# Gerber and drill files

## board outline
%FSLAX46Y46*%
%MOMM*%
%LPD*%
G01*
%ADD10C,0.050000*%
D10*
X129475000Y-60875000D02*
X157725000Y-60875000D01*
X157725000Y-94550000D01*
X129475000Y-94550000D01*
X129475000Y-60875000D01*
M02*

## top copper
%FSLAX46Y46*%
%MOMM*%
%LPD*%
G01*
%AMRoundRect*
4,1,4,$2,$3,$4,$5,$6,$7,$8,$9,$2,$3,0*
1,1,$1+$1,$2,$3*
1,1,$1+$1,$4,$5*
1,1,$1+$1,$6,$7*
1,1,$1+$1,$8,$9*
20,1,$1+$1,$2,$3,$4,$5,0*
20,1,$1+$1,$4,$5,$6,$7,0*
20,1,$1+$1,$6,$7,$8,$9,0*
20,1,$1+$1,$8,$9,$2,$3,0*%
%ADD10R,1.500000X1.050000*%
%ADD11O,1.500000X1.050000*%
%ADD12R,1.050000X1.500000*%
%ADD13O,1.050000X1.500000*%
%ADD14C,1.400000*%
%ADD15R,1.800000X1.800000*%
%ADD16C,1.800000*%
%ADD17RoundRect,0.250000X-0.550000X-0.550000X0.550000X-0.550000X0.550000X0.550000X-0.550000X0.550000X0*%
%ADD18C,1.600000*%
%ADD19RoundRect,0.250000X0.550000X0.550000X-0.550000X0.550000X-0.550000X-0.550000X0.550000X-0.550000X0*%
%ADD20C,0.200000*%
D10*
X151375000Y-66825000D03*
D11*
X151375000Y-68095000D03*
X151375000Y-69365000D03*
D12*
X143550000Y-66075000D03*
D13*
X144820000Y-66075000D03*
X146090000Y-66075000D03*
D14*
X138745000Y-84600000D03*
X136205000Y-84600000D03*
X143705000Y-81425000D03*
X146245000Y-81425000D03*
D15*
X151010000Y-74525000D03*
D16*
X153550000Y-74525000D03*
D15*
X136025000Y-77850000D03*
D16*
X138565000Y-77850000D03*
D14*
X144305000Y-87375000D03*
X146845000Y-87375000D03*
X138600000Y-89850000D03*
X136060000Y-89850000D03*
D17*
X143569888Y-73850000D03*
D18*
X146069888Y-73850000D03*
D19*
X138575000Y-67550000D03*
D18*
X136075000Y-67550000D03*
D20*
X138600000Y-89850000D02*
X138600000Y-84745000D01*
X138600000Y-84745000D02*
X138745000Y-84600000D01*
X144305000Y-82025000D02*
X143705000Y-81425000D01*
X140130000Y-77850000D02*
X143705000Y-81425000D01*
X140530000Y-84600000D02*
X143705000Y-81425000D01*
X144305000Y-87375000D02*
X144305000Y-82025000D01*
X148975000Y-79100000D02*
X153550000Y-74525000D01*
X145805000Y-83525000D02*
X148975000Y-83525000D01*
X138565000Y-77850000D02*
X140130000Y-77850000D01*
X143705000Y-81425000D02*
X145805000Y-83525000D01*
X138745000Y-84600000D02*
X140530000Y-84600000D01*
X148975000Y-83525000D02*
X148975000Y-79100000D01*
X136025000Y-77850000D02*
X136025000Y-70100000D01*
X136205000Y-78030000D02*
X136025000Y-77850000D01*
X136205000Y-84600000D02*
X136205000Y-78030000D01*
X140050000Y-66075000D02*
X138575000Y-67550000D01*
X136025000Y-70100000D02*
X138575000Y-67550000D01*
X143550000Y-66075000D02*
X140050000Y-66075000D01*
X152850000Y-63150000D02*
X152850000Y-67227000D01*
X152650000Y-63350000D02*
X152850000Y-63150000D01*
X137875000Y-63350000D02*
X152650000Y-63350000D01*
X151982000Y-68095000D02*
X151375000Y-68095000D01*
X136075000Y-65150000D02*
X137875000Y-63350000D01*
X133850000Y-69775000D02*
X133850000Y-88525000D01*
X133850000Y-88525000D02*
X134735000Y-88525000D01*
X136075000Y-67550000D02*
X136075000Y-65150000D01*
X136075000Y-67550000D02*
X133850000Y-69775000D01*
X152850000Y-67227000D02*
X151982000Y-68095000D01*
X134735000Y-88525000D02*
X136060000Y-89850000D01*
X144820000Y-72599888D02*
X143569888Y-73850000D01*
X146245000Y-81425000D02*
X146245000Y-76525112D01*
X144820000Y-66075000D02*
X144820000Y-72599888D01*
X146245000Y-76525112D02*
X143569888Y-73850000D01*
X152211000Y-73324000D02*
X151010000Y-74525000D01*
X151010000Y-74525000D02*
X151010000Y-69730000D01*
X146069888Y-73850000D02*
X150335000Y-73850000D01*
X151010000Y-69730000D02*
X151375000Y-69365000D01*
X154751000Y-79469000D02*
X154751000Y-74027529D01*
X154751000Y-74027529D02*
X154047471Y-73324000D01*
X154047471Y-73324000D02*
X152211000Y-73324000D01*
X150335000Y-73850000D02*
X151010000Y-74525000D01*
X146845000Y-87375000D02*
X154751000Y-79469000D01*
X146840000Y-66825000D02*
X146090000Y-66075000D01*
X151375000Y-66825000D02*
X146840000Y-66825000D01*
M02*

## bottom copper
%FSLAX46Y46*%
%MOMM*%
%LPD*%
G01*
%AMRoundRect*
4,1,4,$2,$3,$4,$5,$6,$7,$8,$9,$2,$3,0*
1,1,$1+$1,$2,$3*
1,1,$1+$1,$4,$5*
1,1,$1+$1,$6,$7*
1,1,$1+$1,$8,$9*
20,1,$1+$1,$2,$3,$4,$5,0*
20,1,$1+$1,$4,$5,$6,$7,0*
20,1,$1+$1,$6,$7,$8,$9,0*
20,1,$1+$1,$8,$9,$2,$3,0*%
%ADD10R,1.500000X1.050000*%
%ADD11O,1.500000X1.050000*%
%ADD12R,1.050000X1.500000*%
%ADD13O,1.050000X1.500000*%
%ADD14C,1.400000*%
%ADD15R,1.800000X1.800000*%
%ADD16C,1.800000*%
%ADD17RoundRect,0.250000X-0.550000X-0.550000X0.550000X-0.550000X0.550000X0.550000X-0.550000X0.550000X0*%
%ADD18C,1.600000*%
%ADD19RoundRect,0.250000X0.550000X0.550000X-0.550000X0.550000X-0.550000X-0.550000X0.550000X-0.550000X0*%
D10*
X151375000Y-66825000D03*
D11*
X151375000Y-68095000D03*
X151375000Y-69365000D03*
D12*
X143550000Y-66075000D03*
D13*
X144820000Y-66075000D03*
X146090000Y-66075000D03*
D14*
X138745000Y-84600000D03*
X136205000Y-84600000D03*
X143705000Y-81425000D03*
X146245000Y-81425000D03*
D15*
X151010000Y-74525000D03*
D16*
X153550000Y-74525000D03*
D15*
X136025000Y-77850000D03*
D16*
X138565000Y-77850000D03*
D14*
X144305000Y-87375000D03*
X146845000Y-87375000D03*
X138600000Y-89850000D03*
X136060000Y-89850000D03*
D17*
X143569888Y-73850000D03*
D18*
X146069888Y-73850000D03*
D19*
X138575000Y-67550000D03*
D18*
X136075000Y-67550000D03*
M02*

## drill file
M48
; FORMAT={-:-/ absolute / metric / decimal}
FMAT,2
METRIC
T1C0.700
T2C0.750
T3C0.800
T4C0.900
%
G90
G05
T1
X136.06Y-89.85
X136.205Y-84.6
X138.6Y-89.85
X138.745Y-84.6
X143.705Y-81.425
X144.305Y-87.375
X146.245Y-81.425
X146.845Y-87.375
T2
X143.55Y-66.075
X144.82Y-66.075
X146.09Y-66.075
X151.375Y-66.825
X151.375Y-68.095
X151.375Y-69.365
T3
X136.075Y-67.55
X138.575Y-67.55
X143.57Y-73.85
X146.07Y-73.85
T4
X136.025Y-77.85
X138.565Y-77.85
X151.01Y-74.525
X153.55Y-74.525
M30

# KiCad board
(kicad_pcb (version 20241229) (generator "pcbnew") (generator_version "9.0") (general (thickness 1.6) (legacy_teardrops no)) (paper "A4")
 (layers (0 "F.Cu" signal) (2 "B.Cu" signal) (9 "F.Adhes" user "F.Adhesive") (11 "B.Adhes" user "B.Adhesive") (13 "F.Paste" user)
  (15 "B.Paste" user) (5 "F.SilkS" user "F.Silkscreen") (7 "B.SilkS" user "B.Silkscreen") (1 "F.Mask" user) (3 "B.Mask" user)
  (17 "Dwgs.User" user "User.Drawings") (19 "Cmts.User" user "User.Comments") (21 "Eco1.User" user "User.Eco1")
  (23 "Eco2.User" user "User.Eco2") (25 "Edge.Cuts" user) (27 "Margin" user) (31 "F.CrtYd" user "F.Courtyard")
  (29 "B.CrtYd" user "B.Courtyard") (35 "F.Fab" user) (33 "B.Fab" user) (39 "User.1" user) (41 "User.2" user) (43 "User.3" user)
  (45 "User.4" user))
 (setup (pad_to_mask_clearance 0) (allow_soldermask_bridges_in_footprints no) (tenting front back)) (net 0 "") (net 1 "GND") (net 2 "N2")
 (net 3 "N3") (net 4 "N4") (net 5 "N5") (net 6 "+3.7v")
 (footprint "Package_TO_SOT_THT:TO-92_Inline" (layer "F.Cu") (at 151.375 66.825 -90)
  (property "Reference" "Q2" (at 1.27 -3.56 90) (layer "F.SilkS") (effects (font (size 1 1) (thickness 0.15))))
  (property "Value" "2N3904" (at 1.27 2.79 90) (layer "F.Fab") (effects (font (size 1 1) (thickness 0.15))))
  (pad "1" thru_hole rect (at 0 0 270) (size 1.05 1.5) (drill 0.75) (layers "*.Cu" "*.Mask") (remove_unused_layers no) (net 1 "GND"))
  (pad "2" thru_hole oval (at 1.27 0 270) (size 1.05 1.5) (drill 0.75) (layers "*.Cu" "*.Mask") (remove_unused_layers no) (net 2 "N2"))
  (pad "3" thru_hole oval (at 2.54 0 270) (size 1.05 1.5) (drill 0.75) (layers "*.Cu" "*.Mask") (remove_unused_layers no) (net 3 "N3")))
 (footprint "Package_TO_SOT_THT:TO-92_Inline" (layer "F.Cu") (at 143.55 66.075)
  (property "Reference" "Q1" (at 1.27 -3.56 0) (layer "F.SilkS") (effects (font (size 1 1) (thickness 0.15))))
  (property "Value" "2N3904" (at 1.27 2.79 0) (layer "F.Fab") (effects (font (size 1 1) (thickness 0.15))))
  (pad "1" thru_hole rect (at 0 0) (size 1.05 1.5) (drill 0.75) (layers "*.Cu" "*.Mask") (remove_unused_layers no) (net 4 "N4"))
  (pad "2" thru_hole oval (at 1.27 0) (size 1.05 1.5) (drill 0.75) (layers "*.Cu" "*.Mask") (remove_unused_layers no) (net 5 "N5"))
  (pad "3" thru_hole oval (at 2.54 0) (size 1.05 1.5) (drill 0.75) (layers "*.Cu" "*.Mask") (remove_unused_layers no) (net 1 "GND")))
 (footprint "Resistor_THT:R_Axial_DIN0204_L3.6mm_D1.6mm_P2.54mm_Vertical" (layer "F.Cu") (at 138.745 84.6 180)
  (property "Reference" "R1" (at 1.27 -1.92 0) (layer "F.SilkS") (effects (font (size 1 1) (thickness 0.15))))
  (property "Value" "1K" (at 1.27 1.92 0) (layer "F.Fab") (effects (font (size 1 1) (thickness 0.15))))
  (pad "1" thru_hole circle (at 0 0 180) (size 1.4 1.4) (drill 0.7) (layers "*.Cu" "*.Mask") (remove_unused_layers no) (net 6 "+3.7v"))
  (pad "2" thru_hole circle (at 2.54 0 180) (size 1.4 1.4) (drill 0.7) (layers "*.Cu" "*.Mask") (remove_unused_layers no) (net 4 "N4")))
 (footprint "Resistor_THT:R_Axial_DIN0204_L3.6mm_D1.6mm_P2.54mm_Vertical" (layer "F.Cu") (at 143.705 81.425)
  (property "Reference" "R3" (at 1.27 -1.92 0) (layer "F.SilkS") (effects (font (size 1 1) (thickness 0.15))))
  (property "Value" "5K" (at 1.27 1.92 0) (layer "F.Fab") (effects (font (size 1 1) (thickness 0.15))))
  (pad "1" thru_hole circle (at 0 0) (size 1.4 1.4) (drill 0.7) (layers "*.Cu" "*.Mask") (remove_unused_layers no) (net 6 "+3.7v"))
  (pad "2" thru_hole circle (at 2.54 0) (size 1.4 1.4) (drill 0.7) (layers "*.Cu" "*.Mask") (remove_unused_layers no) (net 5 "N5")))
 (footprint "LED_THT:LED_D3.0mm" (layer "F.Cu") (at 151.01 74.525)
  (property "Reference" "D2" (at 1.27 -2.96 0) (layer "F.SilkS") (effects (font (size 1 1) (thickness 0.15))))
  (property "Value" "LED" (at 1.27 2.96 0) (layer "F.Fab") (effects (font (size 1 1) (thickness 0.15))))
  (pad "1" thru_hole rect (at 0 0) (size 1.8 1.8) (drill 0.9) (layers "*.Cu" "*.Mask") (remove_unused_layers no) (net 3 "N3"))
  (pad "2" thru_hole circle (at 2.54 0) (size 1.8 1.8) (drill 0.9) (layers "*.Cu" "*.Mask") (remove_unused_layers no) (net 6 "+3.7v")))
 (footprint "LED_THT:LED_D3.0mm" (layer "F.Cu") (at 136.025 77.85)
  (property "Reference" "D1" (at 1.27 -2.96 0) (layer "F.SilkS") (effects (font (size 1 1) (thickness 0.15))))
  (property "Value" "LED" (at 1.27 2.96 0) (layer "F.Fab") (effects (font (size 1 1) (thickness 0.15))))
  (pad "1" thru_hole rect (at 0 0) (size 1.8 1.8) (drill 0.9) (layers "*.Cu" "*.Mask") (remove_unused_layers no) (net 4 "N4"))
  (pad "2" thru_hole circle (at 2.54 0) (size 1.8 1.8) (drill 0.9) (layers "*.Cu" "*.Mask") (remove_unused_layers no) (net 6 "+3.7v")))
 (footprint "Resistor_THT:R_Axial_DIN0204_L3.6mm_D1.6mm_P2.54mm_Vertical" (layer "F.Cu") (at 144.305 87.375)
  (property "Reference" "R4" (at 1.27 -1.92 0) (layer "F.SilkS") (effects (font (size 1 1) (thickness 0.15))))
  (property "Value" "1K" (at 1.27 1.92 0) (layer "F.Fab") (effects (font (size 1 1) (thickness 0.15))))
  (pad "1" thru_hole circle (at 0 0) (size 1.4 1.4) (drill 0.7) (layers "*.Cu" "*.Mask") (remove_unused_layers no) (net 6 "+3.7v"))
  (pad "2" thru_hole circle (at 2.54 0) (size 1.4 1.4) (drill 0.7) (layers "*.Cu" "*.Mask") (remove_unused_layers no) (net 3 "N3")))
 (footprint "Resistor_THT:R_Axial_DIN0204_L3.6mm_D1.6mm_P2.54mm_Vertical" (layer "F.Cu") (at 138.6 89.85 180)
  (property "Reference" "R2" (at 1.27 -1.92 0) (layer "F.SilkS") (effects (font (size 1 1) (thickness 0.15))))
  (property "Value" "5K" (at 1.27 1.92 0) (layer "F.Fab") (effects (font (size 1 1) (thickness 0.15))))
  (pad "1" thru_hole circle (at 0 0 180) (size 1.4 1.4) (drill 0.7) (layers "*.Cu" "*.Mask") (remove_unused_layers no) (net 6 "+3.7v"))
  (pad "2" thru_hole circle (at 2.54 0 180) (size 1.4 1.4) (drill 0.7) (layers "*.Cu" "*.Mask") (remove_unused_layers no) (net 2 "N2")))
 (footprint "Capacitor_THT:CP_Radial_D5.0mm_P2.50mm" (layer "F.Cu") (at 143.569888 73.85)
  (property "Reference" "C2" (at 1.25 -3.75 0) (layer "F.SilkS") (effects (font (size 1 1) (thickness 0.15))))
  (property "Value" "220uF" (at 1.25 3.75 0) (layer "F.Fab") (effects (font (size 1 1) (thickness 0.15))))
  (pad "1" thru_hole roundrect (at 0 0) (size 1.6 1.6) (drill 0.8) (layers "*.Cu" "*.Mask") (remove_unused_layers no)
   (roundrect_rratio 0.15625) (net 5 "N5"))
  (pad "2" thru_hole circle (at 2.5 0) (size 1.6 1.6) (drill 0.8) (layers "*.Cu" "*.Mask") (remove_unused_layers no) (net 3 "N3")))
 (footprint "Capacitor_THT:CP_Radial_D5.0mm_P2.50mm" (layer "F.Cu") (at 138.575 67.55 180)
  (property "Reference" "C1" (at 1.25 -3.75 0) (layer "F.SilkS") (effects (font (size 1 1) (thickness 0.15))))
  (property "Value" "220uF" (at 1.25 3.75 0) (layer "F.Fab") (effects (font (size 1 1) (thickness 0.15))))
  (pad "1" thru_hole roundrect (at 0 0 180) (size 1.6 1.6) (drill 0.8) (layers "*.Cu" "*.Mask") (remove_unused_layers no)
   (roundrect_rratio 0.15625) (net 4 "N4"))
  (pad "2" thru_hole circle (at 2.5 0 180) (size 1.6 1.6) (drill 0.8) (layers "*.Cu" "*.Mask") (remove_unused_layers no) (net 2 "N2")))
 (gr_rect (start 129.475 60.875) (end 157.725 94.55) (stroke (width 0.05) (type default)) (fill no) (layer "Edge.Cuts"))
 (segment (start 138.6 89.85) (end 138.6 84.745) (width 0.2) (layer "F.Cu") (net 6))
 (segment (start 138.6 84.745) (end 138.745 84.6) (width 0.2) (layer "F.Cu") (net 6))
 (segment (start 144.305 82.025) (end 143.705 81.425) (width 0.2) (layer "F.Cu") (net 6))
 (segment (start 140.13 77.85) (end 143.705 81.425) (width 0.2) (layer "F.Cu") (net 6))
 (segment (start 140.53 84.6) (end 143.705 81.425) (width 0.2) (layer "F.Cu") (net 6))
 (segment (start 144.305 87.375) (end 144.305 82.025) (width 0.2) (layer "F.Cu") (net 6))
 (segment (start 148.975 79.1) (end 153.55 74.525) (width 0.2) (layer "F.Cu") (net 6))
 (segment (start 145.805 83.525) (end 148.975 83.525) (width 0.2) (layer "F.Cu") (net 6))
 (segment (start 138.565 77.85) (end 140.13 77.85) (width 0.2) (layer "F.Cu") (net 6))
 (segment (start 143.705 81.425) (end 145.805 83.525) (width 0.2) (layer "F.Cu") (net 6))
 (segment (start 138.745 84.6) (end 140.53 84.6) (width 0.2) (layer "F.Cu") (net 6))
 (segment (start 148.975 83.525) (end 148.975 79.1) (width 0.2) (layer "F.Cu") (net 6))
 (segment (start 136.025 77.85) (end 136.025 70.1) (width 0.2) (layer "F.Cu") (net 4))
 (segment (start 136.205 78.03) (end 136.025 77.85) (width 0.2) (layer "F.Cu") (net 4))
 (segment (start 136.205 84.6) (end 136.205 78.03) (width 0.2) (layer "F.Cu") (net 4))
 (segment (start 140.05 66.075) (end 138.575 67.55) (width 0.2) (layer "F.Cu") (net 4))
 (segment (start 136.025 70.1) (end 138.575 67.55) (width 0.2) (layer "F.Cu") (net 4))
 (segment (start 143.55 66.075) (end 140.05 66.075) (width 0.2) (layer "F.Cu") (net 4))
 (segment (start 152.85 63.15) (end 152.85 67.227) (width 0.2) (layer "F.Cu") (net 2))
 (segment (start 152.65 63.35) (end 152.85 63.15) (width 0.2) (layer "F.Cu") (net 2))
 (segment (start 137.875 63.35) (end 152.65 63.35) (width 0.2) (layer "F.Cu") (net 2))
 (segment (start 151.982 68.095) (end 151.375 68.095) (width 0.2) (layer "F.Cu") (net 2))
 (segment (start 136.075 65.15) (end 137.875 63.35) (width 0.2) (layer "F.Cu") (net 2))
 (segment (start 133.85 69.775) (end 133.85 88.525) (width 0.2) (layer "F.Cu") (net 2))
 (segment (start 133.85 88.525) (end 134.735 88.525) (width 0.2) (layer "F.Cu") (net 2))
 (segment (start 136.075 67.55) (end 136.075 65.15) (width 0.2) (layer "F.Cu") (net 2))
 (segment (start 136.075 67.55) (end 133.85 69.775) (width 0.2) (layer "F.Cu") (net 2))
 (segment (start 152.85 67.227) (end 151.982 68.095) (width 0.2) (layer "F.Cu") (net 2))
 (segment (start 134.735 88.525) (end 136.06 89.85) (width 0.2) (layer "F.Cu") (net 2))
 (segment (start 144.82 72.599888) (end 143.569888 73.85) (width 0.2) (layer "F.Cu") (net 5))
 (segment (start 146.245 81.425) (end 146.245 76.525112) (width 0.2) (layer "F.Cu") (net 5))
 (segment (start 144.82 66.075) (end 144.82 72.599888) (width 0.2) (layer "F.Cu") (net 5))
 (segment (start 146.245 76.525112) (end 143.569888 73.85) (width 0.2) (layer "F.Cu") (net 5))
 (segment (start 152.211 73.324) (end 151.01 74.525) (width 0.2) (layer "F.Cu") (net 3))
 (segment (start 151.01 74.525) (end 151.01 69.73) (width 0.2) (layer "F.Cu") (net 3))
 (segment (start 146.069888 73.85) (end 150.335 73.85) (width 0.2) (layer "F.Cu") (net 3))
 (segment (start 151.01 69.73) (end 151.375 69.365) (width 0.2) (layer "F.Cu") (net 3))
 (segment (start 154.751 79.469) (end 154.751 74.027529) (width 0.2) (layer "F.Cu") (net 3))
 (segment (start 154.751 74.027529) (end 154.047471 73.324) (width 0.2) (layer "F.Cu") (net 3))
 (segment (start 154.047471 73.324) (end 152.211 73.324) (width 0.2) (layer "F.Cu") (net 3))
 (segment (start 150.335 73.85) (end 151.01 74.525) (width 0.2) (layer "F.Cu") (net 3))
 (segment (start 146.845 87.375) (end 154.751 79.469) (width 0.2) (layer "F.Cu") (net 3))
 (segment (start 146.84 66.825) (end 146.09 66.075) (width 0.2) (layer "F.Cu") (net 1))
 (segment (start 151.375 66.825) (end 146.84 66.825) (width 0.2) (layer "F.Cu") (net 1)))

